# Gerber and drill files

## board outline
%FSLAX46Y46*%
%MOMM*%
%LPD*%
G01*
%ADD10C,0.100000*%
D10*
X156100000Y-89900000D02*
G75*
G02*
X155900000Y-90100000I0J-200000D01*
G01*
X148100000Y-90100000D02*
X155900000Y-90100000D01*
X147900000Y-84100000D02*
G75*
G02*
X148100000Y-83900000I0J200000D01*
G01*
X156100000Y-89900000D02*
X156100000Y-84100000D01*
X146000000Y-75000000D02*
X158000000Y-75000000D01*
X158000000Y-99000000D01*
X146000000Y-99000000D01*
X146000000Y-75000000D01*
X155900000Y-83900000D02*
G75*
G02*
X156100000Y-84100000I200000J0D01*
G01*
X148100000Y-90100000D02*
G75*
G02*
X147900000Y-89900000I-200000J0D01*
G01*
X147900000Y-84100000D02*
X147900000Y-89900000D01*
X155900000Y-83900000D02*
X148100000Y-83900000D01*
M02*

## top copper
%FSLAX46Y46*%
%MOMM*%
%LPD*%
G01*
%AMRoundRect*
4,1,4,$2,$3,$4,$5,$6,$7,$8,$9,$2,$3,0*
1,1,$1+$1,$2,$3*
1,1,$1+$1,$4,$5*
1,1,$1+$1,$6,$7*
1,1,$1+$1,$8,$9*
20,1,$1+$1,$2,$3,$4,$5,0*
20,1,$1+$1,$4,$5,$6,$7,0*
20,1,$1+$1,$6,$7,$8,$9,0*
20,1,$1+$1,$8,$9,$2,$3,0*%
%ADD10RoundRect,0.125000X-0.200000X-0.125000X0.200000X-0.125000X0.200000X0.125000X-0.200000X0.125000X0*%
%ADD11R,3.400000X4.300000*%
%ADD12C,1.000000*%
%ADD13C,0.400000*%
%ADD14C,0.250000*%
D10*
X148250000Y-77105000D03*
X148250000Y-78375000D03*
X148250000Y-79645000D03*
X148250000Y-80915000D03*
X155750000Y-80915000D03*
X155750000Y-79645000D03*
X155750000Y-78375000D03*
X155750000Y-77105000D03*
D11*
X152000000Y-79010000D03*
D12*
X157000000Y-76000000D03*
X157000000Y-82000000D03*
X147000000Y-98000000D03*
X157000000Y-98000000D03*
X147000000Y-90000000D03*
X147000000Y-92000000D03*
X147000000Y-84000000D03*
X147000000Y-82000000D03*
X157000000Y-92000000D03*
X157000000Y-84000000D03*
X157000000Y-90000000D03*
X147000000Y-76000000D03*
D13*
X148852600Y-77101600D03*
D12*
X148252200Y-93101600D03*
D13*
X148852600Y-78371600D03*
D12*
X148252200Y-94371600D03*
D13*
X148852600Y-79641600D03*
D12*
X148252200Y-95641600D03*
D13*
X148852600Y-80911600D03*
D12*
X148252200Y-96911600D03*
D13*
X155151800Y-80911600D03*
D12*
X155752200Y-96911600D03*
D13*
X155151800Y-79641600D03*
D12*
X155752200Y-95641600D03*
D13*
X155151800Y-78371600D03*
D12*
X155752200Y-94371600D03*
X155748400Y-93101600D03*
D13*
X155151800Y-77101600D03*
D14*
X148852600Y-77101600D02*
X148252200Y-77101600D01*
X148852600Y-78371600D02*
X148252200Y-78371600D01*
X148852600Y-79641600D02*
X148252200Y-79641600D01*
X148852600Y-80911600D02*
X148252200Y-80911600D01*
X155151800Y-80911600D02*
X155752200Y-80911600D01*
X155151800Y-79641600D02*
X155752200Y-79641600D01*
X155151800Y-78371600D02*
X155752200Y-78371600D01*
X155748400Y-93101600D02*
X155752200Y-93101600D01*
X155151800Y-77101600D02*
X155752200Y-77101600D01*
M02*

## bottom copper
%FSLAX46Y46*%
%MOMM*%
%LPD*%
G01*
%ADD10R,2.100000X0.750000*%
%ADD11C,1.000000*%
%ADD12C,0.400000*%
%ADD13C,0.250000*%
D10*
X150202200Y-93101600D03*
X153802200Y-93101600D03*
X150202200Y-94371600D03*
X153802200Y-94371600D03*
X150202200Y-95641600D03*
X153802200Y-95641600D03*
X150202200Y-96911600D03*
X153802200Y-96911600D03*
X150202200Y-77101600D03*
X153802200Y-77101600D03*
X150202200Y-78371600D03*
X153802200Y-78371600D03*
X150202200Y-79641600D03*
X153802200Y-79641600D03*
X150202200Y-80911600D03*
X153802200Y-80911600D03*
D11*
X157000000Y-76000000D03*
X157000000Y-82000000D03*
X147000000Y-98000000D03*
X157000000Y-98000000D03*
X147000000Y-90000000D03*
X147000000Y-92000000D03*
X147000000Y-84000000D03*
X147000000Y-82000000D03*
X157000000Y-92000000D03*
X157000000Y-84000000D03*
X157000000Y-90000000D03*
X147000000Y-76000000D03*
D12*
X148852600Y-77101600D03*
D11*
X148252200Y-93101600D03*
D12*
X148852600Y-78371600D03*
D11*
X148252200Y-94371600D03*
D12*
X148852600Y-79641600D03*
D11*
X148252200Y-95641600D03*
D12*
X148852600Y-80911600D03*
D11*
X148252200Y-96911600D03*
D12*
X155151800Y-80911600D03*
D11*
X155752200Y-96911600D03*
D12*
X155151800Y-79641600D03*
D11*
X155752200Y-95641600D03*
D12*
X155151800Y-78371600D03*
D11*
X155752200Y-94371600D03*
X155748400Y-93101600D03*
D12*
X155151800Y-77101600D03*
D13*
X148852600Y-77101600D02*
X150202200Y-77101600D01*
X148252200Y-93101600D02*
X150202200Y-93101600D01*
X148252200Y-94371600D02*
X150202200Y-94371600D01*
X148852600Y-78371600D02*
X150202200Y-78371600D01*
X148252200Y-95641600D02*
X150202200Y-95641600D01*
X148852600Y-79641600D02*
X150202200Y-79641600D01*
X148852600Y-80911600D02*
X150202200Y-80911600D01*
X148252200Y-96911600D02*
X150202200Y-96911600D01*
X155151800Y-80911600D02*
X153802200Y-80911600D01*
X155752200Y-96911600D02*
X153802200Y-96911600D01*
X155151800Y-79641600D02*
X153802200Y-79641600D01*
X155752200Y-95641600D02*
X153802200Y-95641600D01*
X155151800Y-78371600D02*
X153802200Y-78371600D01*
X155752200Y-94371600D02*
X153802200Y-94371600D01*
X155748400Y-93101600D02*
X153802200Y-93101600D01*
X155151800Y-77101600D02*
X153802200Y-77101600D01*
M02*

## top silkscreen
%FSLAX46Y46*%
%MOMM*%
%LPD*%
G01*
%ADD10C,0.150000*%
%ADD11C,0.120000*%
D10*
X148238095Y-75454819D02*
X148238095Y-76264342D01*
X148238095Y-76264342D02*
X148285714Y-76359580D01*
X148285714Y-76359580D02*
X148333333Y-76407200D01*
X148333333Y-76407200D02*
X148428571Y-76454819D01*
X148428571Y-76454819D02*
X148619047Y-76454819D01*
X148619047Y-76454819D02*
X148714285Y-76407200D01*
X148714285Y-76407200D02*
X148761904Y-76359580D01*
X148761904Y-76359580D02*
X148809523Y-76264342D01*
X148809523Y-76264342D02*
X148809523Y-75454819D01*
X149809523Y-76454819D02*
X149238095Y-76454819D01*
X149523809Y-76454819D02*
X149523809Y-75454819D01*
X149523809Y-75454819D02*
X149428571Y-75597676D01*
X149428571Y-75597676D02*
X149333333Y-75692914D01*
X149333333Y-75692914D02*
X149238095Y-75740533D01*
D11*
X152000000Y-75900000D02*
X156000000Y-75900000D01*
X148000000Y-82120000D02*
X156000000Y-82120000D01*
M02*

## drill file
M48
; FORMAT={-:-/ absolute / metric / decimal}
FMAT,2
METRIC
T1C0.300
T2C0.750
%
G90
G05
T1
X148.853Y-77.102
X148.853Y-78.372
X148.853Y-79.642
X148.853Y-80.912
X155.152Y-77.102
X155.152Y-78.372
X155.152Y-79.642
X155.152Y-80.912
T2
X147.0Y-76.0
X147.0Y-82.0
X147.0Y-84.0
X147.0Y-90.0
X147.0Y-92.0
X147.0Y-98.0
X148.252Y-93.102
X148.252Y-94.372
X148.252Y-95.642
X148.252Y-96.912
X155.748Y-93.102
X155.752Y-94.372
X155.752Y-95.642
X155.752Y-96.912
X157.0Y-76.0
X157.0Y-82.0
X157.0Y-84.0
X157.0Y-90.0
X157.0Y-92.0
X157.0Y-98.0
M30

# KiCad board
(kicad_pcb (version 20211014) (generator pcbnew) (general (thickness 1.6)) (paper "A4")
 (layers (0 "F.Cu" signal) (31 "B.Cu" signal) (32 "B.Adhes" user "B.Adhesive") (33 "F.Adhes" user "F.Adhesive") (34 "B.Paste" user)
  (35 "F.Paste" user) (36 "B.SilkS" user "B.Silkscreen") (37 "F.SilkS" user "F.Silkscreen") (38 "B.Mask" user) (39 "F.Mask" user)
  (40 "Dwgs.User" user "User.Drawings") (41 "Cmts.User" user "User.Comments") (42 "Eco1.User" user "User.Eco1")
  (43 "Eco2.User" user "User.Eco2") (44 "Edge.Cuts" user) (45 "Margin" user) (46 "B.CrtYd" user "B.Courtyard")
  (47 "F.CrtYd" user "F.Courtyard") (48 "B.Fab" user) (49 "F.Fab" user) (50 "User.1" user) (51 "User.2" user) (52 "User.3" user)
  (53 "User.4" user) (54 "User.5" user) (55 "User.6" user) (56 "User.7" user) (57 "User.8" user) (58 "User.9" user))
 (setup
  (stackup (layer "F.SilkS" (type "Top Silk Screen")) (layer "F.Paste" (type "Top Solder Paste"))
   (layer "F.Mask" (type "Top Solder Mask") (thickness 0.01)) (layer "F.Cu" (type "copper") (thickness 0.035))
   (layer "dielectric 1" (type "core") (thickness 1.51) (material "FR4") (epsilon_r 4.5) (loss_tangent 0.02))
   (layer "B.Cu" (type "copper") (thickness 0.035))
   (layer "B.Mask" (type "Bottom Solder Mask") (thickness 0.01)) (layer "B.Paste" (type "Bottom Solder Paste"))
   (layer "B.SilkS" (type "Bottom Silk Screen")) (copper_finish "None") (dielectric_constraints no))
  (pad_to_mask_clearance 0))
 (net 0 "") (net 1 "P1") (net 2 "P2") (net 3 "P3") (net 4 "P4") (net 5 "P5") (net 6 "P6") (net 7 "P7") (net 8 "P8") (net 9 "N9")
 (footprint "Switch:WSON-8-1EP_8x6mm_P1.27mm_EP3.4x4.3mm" (layer "F.Cu") (at 156 76)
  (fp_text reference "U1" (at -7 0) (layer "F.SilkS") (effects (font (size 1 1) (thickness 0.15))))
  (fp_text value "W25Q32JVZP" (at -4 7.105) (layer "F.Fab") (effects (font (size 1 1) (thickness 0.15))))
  (fp_line (start -4 -0.1) (end 0 -0.1) (layer "F.SilkS") (width 0.12))
  (fp_line (start -8 6.12) (end 0 6.12) (layer "F.SilkS") (width 0.12))
  (pad "" smd roundrect (at -3.15 4.085) (size 1.37 1.73) (layers "F.Paste") (roundrect_rratio 0.182482))
  (pad "" smd roundrect (at -4.85 4.085) (size 1.37 1.73) (layers "F.Paste") (roundrect_rratio 0.182482))
  (pad "" smd roundrect (at -3.15 1.935) (size 1.37 1.73) (layers "F.Paste") (roundrect_rratio 0.182482))
  (pad "" smd roundrect (at -4.85 1.935) (size 1.37 1.73) (layers "F.Paste") (roundrect_rratio 0.182482))
  (pad "1" smd roundrect (at -7.75 1.105) (size 0.65 0.5) (layers "F.Cu" "F.Paste" "F.Mask") (roundrect_rratio 0.25) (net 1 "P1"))
  (pad "2" smd roundrect (at -7.75 2.375) (size 0.65 0.5) (layers "F.Cu" "F.Paste" "F.Mask") (roundrect_rratio 0.25) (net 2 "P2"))
  (pad "3" smd roundrect (at -7.75 3.645) (size 0.65 0.5) (layers "F.Cu" "F.Paste" "F.Mask") (roundrect_rratio 0.25) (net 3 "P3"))
  (pad "4" smd roundrect (at -7.75 4.915) (size 0.65 0.5) (layers "F.Cu" "F.Paste" "F.Mask") (roundrect_rratio 0.25) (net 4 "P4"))
  (pad "5" smd roundrect (at -0.25 4.915) (size 0.65 0.5) (layers "F.Cu" "F.Paste" "F.Mask") (roundrect_rratio 0.25) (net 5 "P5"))
  (pad "6" smd roundrect (at -0.25 3.645) (size 0.65 0.5) (layers "F.Cu" "F.Paste" "F.Mask") (roundrect_rratio 0.25) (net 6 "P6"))
  (pad "7" smd roundrect (at -0.25 2.375) (size 0.65 0.5) (layers "F.Cu" "F.Paste" "F.Mask") (roundrect_rratio 0.25) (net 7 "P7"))
  (pad "8" smd roundrect (at -0.25 1.105) (size 0.65 0.5) (layers "F.Cu" "F.Paste" "F.Mask") (roundrect_rratio 0.25) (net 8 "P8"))
  (pad "9" smd rect (at -4 3.01) (size 3.4 4.3) (layers "F.Cu" "F.Mask") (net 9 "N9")))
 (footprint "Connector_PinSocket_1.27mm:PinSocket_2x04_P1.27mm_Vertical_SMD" (layer "B.Cu") (at 152.0022 95.0066 180)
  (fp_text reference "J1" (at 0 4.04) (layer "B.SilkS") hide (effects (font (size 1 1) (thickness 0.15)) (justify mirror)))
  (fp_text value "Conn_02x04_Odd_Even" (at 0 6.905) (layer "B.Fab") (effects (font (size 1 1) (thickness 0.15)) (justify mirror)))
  (pad "1" smd rect (at 1.8 1.905 180) (size 2.1 0.75) (layers "B.Cu" "B.Paste" "B.Mask") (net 1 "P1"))
  (pad "2" smd rect (at -1.8 1.905 180) (size 2.1 0.75) (layers "B.Cu" "B.Paste" "B.Mask") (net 8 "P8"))
  (pad "3" smd rect (at 1.8 0.635 180) (size 2.1 0.75) (layers "B.Cu" "B.Paste" "B.Mask") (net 2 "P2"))
  (pad "4" smd rect (at -1.8 0.635 180) (size 2.1 0.75) (layers "B.Cu" "B.Paste" "B.Mask") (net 7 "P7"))
  (pad "5" smd rect (at 1.8 -0.635 180) (size 2.1 0.75) (layers "B.Cu" "B.Paste" "B.Mask") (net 3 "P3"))
  (pad "6" smd rect (at -1.8 -0.635 180) (size 2.1 0.75) (layers "B.Cu" "B.Paste" "B.Mask") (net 6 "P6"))
  (pad "7" smd rect (at 1.8 -1.905 180) (size 2.1 0.75) (layers "B.Cu" "B.Paste" "B.Mask") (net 4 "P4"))
  (pad "8" smd rect (at -1.8 -1.905 180) (size 2.1 0.75) (layers "B.Cu" "B.Paste" "B.Mask") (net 5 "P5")))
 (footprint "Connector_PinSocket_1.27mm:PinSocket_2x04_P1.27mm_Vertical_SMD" (layer "B.Cu") (at 152.0022 79.0066 180)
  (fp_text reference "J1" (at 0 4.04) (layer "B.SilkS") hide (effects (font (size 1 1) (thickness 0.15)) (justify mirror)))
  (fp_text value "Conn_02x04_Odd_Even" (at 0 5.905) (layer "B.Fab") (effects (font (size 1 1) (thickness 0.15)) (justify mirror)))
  (pad "1" smd rect (at 1.8 1.905 180) (size 2.1 0.75) (layers "B.Cu" "B.Paste" "B.Mask") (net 1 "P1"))
  (pad "2" smd rect (at -1.8 1.905 180) (size 2.1 0.75) (layers "B.Cu" "B.Paste" "B.Mask") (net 8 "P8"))
  (pad "3" smd rect (at 1.8 0.635 180) (size 2.1 0.75) (layers "B.Cu" "B.Paste" "B.Mask") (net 2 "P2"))
  (pad "4" smd rect (at -1.8 0.635 180) (size 2.1 0.75) (layers "B.Cu" "B.Paste" "B.Mask") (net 7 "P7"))
  (pad "5" smd rect (at 1.8 -0.635 180) (size 2.1 0.75) (layers "B.Cu" "B.Paste" "B.Mask") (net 3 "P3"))
  (pad "6" smd rect (at -1.8 -0.635 180) (size 2.1 0.75) (layers "B.Cu" "B.Paste" "B.Mask") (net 6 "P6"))
  (pad "7" smd rect (at 1.8 -1.905 180) (size 2.1 0.75) (layers "B.Cu" "B.Paste" "B.Mask") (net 4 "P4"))
  (pad "8" smd rect (at -1.8 -1.905 180) (size 2.1 0.75) (layers "B.Cu" "B.Paste" "B.Mask") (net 5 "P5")))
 (gr_arc (start 156.1 89.9) (mid 156.241421 90.241421) (end 155.9 90.1) (layer "Edge.Cuts") (width 0.1))
 (gr_line (start 148.1 90.1) (end 155.9 90.1) (layer "Edge.Cuts") (width 0.1))
 (gr_arc (start 147.9 84.1) (mid 147.758579 83.758579) (end 148.1 83.9) (layer "Edge.Cuts") (width 0.1))
 (gr_line (start 156.1 89.9) (end 156.1 84.1) (layer "Edge.Cuts") (width 0.1))
 (gr_rect (start 146 75) (end 158 99) (layer "Edge.Cuts") (width 0.1) (fill none))
 (gr_arc (start 155.9 83.9) (mid 156.241421 83.758579) (end 156.1 84.1) (layer "Edge.Cuts") (width 0.1))
 (gr_arc (start 148.1 90.1) (mid 147.758579 90.241421) (end 147.9 89.9) (layer "Edge.Cuts") (width 0.1))
 (gr_line (start 147.9 84.1) (end 147.9 89.9) (layer "Edge.Cuts") (width 0.1))
 (gr_line (start 155.9 83.9) (end 148.1 83.9) (layer "Edge.Cuts") (width 0.1))
 (via (at 157 76) (size 1) (drill 0.75) (layers "F.Cu" "B.Cu") (free) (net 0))
 (via (at 157 82) (size 1) (drill 0.75) (layers "F.Cu" "B.Cu") (free) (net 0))
 (via (at 147 98) (size 1) (drill 0.75) (layers "F.Cu" "B.Cu") (free) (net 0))
 (via (at 157 98) (size 1) (drill 0.75) (layers "F.Cu" "B.Cu") (free) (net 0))
 (via (at 147 90) (size 1) (drill 0.75) (layers "F.Cu" "B.Cu") (free) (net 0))
 (via (at 147 92) (size 1) (drill 0.75) (layers "F.Cu" "B.Cu") (free) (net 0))
 (via (at 147 84) (size 1) (drill 0.75) (layers "F.Cu" "B.Cu") (free) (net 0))
 (via (at 147 82) (size 1) (drill 0.75) (layers "F.Cu" "B.Cu") (free) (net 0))
 (via (at 157 92) (size 1) (drill 0.75) (layers "F.Cu" "B.Cu") (free) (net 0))
 (via (at 157 84) (size 1) (drill 0.75) (layers "F.Cu" "B.Cu") (free) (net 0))
 (via (at 157 90) (size 1) (drill 0.75) (layers "F.Cu" "B.Cu") (free) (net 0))
 (via (at 147 76) (size 1) (drill 0.75) (layers "F.Cu" "B.Cu") (free) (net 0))
 (segment (start 148.8526 77.1016) (end 148.2522 77.1016) (width 0.25) (layer "F.Cu") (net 1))
 (via (at 148.8526 77.1016) (size 0.4) (drill 0.3) (layers "F.Cu" "B.Cu") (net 1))
 (via (at 148.2522 93.1016) (size 1) (drill 0.75) (layers "F.Cu" "B.Cu") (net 1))
 (segment (start 148.8526 77.1016) (end 150.2022 77.1016) (width 0.25) (layer "B.Cu") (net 1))
 (segment (start 148.2522 93.1016) (end 150.2022 93.1016) (width 0.25) (layer "B.Cu") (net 1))
 (segment (start 148.8526 78.3716) (end 148.2522 78.3716) (width 0.25) (layer "F.Cu") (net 2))
 (via (at 148.8526 78.3716) (size 0.4) (drill 0.3) (layers "F.Cu" "B.Cu") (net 2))
 (via (at 148.2522 94.3716) (size 1) (drill 0.75) (layers "F.Cu" "B.Cu") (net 2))
 (segment (start 148.2522 94.3716) (end 150.2022 94.3716) (width 0.25) (layer "B.Cu") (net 2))
 (segment (start 148.8526 78.3716) (end 150.2022 78.3716) (width 0.25) (layer "B.Cu") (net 2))
 (segment (start 148.8526 79.6416) (end 148.2522 79.6416) (width 0.25) (layer "F.Cu") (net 3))
 (via (at 148.8526 79.6416) (size 0.4) (drill 0.3) (layers "F.Cu" "B.Cu") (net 3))
 (via (at 148.2522 95.6416) (size 1) (drill 0.75) (layers "F.Cu" "B.Cu") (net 3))
 (segment (start 148.2522 95.6416) (end 150.2022 95.6416) (width 0.25) (layer "B.Cu") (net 3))
 (segment (start 148.8526 79.6416) (end 150.2022 79.6416) (width 0.25) (layer "B.Cu") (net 3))
 (segment (start 148.8526 80.9116) (end 148.2522 80.9116) (width 0.25) (layer "F.Cu") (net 4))
 (via (at 148.8526 80.9116) (size 0.4) (drill 0.3) (layers "F.Cu" "B.Cu") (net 4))
 (via (at 148.2522 96.9116) (size 1) (drill 0.75) (layers "F.Cu" "B.Cu") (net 4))
 (segment (start 148.8526 80.9116) (end 150.2022 80.9116) (width 0.25) (layer "B.Cu") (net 4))
 (segment (start 148.2522 96.9116) (end 150.2022 96.9116) (width 0.25) (layer "B.Cu") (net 4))
 (segment (start 155.1518 80.9116) (end 155.7522 80.9116) (width 0.25) (layer "F.Cu") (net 5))
 (via (at 155.1518 80.9116) (size 0.4) (drill 0.3) (layers "F.Cu" "B.Cu") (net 5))
 (via (at 155.7522 96.9116) (size 1) (drill 0.75) (layers "F.Cu" "B.Cu") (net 5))
 (segment (start 155.1518 80.9116) (end 153.8022 80.9116) (width 0.25) (layer "B.Cu") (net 5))
 (segment (start 155.7522 96.9116) (end 153.8022 96.9116) (width 0.25) (layer "B.Cu") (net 5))
 (segment (start 155.1518 79.6416) (end 155.7522 79.6416) (width 0.25) (layer "F.Cu") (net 6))
 (via (at 155.1518 79.6416) (size 0.4) (drill 0.3) (layers "F.Cu" "B.Cu") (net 6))
 (via (at 155.7522 95.6416) (size 1) (drill 0.75) (layers "F.Cu" "B.Cu") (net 6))
 (segment (start 155.1518 79.6416) (end 153.8022 79.6416) (width 0.25) (layer "B.Cu") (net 6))
 (segment (start 155.7522 95.6416) (end 153.8022 95.6416) (width 0.25) (layer "B.Cu") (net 6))
 (segment (start 155.1518 78.3716) (end 155.7522 78.3716) (width 0.25) (layer "F.Cu") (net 7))
 (via (at 155.1518 78.3716) (size 0.4) (drill 0.3) (layers "F.Cu" "B.Cu") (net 7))
 (via (at 155.7522 94.3716) (size 1) (drill 0.75) (layers "F.Cu" "B.Cu") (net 7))
 (segment (start 155.1518 78.3716) (end 153.8022 78.3716) (width 0.25) (layer "B.Cu") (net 7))
 (segment (start 155.7522 94.3716) (end 153.8022 94.3716) (width 0.25) (layer "B.Cu") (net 7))
 (segment (start 155.7484 93.1016) (end 155.7522 93.1016) (width 0.25) (layer "F.Cu") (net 8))
 (segment (start 155.1518 77.1016) (end 155.7522 77.1016) (width 0.25) (layer "F.Cu") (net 8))
 (via (at 155.7484 93.1016) (size 1) (drill 0.75) (layers "F.Cu" "B.Cu") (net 8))
 (via (at 155.1518 77.1016) (size 0.4) (drill 0.3) (layers "F.Cu" "B.Cu") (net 8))
 (segment (start 155.7484 93.1016) (end 153.8022 93.1016) (width 0.25) (layer "B.Cu") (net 8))
 (segment (start 155.1518 77.1016) (end 153.8022 77.1016) (width 0.25) (layer "B.Cu") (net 8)))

